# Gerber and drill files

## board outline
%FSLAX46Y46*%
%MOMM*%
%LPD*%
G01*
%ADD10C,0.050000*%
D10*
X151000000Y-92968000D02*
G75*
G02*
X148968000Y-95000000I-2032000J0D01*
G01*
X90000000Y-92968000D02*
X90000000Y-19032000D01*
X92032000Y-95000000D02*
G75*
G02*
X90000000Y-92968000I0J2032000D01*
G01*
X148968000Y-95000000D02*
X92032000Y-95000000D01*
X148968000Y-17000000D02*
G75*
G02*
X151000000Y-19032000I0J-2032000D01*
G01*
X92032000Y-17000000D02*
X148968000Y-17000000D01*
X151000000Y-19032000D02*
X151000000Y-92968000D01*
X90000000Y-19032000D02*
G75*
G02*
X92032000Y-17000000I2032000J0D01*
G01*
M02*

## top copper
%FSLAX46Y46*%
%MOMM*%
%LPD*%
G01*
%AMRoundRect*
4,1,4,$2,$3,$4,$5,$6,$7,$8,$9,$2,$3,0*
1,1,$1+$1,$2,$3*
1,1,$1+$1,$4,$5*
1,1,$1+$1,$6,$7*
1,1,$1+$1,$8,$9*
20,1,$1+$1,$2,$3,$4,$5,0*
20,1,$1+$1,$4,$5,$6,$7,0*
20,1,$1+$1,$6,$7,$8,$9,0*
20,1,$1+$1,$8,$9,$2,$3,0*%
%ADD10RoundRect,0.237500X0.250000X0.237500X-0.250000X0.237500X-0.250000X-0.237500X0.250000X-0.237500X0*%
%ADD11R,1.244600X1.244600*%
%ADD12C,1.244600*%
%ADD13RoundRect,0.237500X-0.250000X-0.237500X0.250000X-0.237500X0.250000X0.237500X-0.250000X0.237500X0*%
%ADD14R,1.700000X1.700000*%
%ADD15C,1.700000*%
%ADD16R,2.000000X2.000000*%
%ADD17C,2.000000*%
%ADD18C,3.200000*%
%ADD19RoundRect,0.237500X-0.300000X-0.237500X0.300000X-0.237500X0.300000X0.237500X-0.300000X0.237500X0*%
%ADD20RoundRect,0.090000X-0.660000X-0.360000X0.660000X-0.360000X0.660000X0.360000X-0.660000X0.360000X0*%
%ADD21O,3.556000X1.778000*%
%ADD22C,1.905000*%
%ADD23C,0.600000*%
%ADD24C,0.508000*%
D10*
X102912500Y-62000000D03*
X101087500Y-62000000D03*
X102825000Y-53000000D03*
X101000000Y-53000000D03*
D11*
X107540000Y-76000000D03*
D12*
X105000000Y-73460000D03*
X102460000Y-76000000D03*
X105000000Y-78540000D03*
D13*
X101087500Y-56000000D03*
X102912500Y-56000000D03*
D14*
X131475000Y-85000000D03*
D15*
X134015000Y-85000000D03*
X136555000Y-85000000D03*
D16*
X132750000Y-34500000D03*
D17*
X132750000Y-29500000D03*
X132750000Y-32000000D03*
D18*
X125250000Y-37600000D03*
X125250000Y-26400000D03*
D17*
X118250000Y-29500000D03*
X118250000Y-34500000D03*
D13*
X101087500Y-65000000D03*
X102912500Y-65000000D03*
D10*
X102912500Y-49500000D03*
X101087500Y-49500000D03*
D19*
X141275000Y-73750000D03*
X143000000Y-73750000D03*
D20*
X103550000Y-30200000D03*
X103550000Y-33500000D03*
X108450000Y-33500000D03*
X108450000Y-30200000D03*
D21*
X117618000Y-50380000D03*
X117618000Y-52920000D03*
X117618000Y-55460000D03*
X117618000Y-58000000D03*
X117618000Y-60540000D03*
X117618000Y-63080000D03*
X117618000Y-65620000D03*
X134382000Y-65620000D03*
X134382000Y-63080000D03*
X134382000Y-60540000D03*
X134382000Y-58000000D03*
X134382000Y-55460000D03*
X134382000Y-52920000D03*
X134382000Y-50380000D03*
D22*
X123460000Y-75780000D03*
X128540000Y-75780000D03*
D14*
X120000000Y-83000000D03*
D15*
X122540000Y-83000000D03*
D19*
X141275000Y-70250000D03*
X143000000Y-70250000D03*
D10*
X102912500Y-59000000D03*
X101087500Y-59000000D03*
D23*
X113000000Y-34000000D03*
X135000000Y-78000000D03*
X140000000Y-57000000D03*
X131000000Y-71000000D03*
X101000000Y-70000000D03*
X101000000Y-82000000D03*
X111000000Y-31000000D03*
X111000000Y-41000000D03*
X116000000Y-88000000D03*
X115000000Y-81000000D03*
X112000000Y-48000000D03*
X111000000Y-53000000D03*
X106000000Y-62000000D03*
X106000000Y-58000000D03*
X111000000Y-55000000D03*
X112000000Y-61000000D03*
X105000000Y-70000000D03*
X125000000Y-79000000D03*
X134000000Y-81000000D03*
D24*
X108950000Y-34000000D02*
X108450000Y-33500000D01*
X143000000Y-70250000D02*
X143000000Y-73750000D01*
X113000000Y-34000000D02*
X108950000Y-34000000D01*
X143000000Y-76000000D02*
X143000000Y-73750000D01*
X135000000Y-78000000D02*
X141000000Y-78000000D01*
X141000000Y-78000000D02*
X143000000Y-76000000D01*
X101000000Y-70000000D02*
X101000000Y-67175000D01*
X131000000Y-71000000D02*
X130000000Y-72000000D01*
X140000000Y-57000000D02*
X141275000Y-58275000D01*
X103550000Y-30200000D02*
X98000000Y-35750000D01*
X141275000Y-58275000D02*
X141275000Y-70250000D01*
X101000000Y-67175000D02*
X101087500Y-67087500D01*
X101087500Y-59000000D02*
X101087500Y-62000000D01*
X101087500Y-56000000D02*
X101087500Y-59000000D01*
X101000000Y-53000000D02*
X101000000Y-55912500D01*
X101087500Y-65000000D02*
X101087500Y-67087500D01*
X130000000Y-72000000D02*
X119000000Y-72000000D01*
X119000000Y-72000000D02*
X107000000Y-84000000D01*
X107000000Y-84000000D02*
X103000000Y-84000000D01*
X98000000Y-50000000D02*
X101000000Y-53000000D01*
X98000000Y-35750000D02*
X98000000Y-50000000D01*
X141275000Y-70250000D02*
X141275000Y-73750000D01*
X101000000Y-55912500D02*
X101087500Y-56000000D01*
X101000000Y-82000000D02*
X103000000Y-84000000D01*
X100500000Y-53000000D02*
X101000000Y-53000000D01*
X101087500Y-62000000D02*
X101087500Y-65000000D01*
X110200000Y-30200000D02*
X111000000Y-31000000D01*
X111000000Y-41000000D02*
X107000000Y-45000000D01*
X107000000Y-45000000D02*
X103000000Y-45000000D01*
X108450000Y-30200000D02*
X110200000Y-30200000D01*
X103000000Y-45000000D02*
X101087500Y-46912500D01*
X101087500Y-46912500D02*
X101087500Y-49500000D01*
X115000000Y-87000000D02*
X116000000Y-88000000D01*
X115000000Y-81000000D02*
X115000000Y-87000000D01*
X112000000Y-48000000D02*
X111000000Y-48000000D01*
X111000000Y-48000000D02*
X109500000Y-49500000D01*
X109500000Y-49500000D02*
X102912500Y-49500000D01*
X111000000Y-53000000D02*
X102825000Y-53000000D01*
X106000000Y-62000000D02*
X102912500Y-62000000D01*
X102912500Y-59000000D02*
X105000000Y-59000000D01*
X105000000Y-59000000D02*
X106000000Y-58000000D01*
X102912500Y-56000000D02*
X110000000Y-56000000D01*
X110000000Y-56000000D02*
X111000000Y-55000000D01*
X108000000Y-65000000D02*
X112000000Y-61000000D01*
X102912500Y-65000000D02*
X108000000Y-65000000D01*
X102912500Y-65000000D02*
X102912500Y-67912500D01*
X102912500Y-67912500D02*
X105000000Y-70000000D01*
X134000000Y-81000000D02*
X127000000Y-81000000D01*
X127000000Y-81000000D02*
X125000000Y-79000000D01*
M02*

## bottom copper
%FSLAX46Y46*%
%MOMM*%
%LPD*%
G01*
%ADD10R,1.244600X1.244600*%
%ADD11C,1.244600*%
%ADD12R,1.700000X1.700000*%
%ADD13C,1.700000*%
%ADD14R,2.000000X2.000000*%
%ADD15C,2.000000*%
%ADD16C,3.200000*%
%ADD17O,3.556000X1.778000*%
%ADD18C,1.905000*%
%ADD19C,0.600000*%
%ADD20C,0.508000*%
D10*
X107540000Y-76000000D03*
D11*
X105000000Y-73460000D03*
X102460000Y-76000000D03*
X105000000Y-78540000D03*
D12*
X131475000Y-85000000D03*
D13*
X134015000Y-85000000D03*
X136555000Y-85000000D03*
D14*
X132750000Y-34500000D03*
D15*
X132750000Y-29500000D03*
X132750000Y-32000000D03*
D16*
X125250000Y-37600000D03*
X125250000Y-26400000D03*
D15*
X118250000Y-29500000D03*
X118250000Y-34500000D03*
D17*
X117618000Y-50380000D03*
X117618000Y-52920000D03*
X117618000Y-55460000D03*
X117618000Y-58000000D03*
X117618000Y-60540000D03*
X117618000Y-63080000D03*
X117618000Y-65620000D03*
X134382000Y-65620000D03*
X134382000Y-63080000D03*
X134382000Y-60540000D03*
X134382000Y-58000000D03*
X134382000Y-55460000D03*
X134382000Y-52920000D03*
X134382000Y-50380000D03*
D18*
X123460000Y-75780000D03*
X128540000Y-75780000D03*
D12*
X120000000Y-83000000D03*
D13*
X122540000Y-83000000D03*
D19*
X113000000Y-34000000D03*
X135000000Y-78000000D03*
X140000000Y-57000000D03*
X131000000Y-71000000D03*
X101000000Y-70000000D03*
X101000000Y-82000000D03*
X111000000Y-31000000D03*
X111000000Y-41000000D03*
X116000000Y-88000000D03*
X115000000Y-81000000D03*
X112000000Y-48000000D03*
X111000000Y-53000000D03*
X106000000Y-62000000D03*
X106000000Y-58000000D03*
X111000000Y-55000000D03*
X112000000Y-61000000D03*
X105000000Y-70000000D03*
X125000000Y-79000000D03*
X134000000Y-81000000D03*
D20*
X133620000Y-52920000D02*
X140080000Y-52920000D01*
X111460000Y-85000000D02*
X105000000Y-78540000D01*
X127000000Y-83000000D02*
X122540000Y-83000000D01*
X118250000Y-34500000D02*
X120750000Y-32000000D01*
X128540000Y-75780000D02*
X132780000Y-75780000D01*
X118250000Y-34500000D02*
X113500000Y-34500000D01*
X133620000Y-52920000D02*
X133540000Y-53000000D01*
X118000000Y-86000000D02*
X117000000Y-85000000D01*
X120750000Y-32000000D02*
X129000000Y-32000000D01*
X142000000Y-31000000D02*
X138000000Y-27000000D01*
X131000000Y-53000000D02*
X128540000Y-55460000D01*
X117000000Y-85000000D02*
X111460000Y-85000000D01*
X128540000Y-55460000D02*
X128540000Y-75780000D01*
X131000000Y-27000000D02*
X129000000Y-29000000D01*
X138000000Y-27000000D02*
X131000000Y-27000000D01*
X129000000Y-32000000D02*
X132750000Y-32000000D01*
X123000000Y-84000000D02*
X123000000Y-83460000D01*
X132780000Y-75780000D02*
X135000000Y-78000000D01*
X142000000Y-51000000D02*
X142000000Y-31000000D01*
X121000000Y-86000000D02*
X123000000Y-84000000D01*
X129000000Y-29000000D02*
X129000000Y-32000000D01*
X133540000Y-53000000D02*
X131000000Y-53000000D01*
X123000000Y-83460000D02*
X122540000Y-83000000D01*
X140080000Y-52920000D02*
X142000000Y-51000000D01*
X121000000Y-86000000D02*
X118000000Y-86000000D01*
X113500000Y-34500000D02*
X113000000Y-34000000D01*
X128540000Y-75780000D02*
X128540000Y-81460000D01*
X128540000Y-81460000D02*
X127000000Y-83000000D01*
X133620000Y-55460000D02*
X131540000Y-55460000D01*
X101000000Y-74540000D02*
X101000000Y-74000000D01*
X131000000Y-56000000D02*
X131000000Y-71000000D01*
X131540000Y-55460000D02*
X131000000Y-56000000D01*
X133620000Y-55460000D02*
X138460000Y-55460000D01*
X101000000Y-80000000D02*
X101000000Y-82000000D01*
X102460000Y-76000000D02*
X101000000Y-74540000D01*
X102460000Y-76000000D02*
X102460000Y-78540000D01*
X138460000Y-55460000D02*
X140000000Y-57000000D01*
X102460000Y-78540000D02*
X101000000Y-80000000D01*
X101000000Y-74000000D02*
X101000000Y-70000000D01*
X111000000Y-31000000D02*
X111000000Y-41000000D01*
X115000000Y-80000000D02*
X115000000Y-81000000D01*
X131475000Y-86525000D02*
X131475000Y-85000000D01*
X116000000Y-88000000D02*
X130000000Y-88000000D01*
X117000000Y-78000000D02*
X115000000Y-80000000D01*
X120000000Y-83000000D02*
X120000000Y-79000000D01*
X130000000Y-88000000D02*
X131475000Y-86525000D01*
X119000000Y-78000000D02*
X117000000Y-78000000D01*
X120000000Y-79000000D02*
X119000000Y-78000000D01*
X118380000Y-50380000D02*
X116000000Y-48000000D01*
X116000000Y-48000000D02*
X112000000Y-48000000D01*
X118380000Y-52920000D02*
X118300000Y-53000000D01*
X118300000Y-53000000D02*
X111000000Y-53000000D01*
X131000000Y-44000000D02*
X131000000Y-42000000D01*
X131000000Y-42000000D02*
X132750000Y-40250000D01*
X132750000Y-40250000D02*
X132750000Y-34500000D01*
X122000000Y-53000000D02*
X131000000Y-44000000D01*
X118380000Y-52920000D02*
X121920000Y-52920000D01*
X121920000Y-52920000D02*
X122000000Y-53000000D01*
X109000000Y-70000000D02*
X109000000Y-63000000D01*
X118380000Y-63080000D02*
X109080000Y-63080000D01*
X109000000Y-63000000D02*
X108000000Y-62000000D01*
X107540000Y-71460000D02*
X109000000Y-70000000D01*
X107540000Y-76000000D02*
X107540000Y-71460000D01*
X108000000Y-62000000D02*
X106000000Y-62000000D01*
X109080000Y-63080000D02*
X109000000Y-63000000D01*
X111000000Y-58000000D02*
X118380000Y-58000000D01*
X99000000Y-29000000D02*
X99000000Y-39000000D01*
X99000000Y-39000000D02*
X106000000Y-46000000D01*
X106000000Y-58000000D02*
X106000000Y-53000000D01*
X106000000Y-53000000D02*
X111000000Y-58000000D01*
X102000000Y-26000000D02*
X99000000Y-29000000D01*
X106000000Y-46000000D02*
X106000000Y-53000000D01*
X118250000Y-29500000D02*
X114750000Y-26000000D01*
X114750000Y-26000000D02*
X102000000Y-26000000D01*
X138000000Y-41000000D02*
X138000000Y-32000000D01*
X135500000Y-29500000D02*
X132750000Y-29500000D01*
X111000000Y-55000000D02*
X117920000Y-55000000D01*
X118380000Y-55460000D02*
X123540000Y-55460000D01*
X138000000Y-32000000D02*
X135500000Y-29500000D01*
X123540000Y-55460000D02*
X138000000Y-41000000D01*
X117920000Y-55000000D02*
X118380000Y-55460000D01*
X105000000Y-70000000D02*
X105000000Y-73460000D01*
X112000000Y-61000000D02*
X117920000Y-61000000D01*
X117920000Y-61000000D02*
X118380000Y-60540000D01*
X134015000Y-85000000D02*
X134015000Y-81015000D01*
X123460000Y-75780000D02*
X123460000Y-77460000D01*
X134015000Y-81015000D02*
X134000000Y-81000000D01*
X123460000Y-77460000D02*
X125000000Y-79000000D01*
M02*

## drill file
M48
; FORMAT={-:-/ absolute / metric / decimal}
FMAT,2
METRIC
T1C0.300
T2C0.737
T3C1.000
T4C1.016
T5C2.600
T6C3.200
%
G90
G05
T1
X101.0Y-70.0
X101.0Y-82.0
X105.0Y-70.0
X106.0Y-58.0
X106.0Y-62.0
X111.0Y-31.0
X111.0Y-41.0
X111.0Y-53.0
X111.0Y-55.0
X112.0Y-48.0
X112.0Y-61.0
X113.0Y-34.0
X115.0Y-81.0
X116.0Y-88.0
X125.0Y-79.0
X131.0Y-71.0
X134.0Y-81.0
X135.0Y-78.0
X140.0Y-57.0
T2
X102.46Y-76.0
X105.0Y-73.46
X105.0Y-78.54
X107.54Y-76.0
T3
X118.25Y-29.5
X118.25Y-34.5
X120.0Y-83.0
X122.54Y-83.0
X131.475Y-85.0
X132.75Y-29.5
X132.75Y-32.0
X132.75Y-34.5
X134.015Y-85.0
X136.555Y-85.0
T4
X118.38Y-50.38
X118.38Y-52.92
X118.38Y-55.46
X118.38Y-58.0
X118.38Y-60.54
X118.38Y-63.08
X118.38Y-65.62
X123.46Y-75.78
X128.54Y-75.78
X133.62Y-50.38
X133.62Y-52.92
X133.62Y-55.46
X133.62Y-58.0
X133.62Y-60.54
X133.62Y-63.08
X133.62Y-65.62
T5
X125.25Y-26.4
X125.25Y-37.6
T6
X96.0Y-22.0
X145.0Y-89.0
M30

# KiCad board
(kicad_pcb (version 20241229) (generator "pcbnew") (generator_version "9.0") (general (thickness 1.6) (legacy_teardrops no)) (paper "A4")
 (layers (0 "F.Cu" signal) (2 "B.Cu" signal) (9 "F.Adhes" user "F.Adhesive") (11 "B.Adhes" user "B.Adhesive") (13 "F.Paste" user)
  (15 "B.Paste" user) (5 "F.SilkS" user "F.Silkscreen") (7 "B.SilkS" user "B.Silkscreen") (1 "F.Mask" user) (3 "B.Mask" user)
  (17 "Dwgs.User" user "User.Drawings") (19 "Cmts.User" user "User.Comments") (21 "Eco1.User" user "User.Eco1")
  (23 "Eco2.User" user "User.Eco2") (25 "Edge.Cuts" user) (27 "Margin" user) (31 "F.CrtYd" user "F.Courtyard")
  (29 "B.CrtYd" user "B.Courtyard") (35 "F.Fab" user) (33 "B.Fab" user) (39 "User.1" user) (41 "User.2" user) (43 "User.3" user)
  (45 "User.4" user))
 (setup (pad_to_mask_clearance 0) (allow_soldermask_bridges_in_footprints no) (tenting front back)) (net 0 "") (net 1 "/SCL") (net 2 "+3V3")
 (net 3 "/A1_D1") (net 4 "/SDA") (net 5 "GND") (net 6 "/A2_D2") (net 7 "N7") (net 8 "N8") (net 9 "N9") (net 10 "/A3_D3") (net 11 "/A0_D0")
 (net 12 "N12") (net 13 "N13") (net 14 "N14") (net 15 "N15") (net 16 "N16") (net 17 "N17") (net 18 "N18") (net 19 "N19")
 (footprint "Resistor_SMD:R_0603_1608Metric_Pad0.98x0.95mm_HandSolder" (layer "F.Cu") (at 102 62 180)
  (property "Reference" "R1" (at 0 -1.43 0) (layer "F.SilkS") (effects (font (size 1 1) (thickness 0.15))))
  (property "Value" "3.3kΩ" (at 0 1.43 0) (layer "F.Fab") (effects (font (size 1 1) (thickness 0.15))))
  (pad "1" smd roundrect (at -0.9125 0 180) (size 0.975 0.95) (layers "F.Cu" "F.Mask" "F.Paste") (roundrect_rratio 0.25) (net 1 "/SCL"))
  (pad "2" smd roundrect (at 0.9125 0 180) (size 0.975 0.95) (layers "F.Cu" "F.Mask" "F.Paste") (roundrect_rratio 0.25) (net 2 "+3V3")))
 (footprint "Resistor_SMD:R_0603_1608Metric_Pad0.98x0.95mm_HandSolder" (layer "F.Cu") (at 101.9125 53 180)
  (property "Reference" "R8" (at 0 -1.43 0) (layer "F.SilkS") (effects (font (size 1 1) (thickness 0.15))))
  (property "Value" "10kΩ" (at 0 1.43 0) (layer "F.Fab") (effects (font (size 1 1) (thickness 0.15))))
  (pad "1" smd roundrect (at -0.9125 0 180) (size 0.975 0.95) (layers "F.Cu" "F.Mask" "F.Paste") (roundrect_rratio 0.25) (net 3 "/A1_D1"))
  (pad "2" smd roundrect (at 0.9125 0 180) (size 0.975 0.95) (layers "F.Cu" "F.Mask" "F.Paste") (roundrect_rratio 0.25) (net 2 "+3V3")))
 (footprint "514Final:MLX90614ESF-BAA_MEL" (layer "F.Cu") (at 107.54 76 90)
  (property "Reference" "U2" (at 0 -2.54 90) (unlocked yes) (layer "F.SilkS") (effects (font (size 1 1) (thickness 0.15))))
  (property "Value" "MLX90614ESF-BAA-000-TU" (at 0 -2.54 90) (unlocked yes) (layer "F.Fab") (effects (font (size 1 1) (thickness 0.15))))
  (pad "1" thru_hole rect (at 0 0 90) (size 1.2446 1.2446) (drill 0.7366) (layers "*.Cu" "*.Mask") (remove_unused_layers no) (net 1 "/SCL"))
  (pad "2" thru_hole circle (at 2.54 -2.54 180) (size 1.2446 1.2446) (drill 0.7366) (layers "*.Cu" "*.Mask") (remove_unused_layers no)
   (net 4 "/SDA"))
  (pad "3" thru_hole circle (at 0 -5.08 90) (size 1.2446 1.2446) (drill 0.7366) (layers "*.Cu" "*.Mask") (remove_unused_layers no)
   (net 2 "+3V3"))
  (pad "4" thru_hole circle (at -2.54 -2.54 180) (size 1.2446 1.2446) (drill 0.7366) (layers "*.Cu" "*.Mask") (remove_unused_layers no)
   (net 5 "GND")))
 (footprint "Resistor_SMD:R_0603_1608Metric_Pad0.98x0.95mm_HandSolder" (layer "F.Cu") (at 102 56)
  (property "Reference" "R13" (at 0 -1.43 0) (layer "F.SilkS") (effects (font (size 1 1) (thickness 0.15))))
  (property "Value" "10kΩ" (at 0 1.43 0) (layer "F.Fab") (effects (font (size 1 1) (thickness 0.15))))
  (pad "1" smd roundrect (at -0.9125 0) (size 0.975 0.95) (layers "F.Cu" "F.Mask" "F.Paste") (roundrect_rratio 0.25) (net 2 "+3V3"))
  (pad "2" smd roundrect (at 0.9125 0) (size 0.975 0.95) (layers "F.Cu" "F.Mask" "F.Paste") (roundrect_rratio 0.25) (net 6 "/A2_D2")))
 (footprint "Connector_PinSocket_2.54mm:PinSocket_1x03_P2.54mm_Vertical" (layer "F.Cu") (at 131.475 85 90)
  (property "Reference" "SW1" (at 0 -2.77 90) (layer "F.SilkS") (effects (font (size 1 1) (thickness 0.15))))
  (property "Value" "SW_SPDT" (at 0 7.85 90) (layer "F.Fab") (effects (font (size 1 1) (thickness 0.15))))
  (pad "1" thru_hole rect (at 0 0 90) (size 1.7 1.7) (drill 1) (layers "*.Cu" "*.Mask") (remove_unused_layers no) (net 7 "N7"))
  (pad "2" thru_hole circle (at 0 2.54 90) (size 1.7 1.7) (drill 1) (layers "*.Cu" "*.Mask") (remove_unused_layers no) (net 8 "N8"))
  (pad "3" thru_hole circle (at 0 5.08 90) (size 1.7 1.7) (drill 1) (layers "*.Cu" "*.Mask") (remove_unused_layers no) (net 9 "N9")))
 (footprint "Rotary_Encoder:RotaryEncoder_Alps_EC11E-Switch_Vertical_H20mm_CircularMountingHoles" (layer "F.Cu") (at 132.75 34.5 180)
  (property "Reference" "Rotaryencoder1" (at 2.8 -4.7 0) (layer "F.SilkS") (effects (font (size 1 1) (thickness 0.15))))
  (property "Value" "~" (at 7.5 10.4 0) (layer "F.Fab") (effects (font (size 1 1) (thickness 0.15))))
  (pad "A" thru_hole rect (at 0 0 180) (size 2 2) (drill 1) (layers "*.Cu" "*.Mask") (remove_unused_layers no) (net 3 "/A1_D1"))
  (pad "B" thru_hole circle (at 0 5 180) (size 2 2) (drill 1) (layers "*.Cu" "*.Mask") (remove_unused_layers no) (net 6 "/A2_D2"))
  (pad "C" thru_hole circle (at 0 2.5 180) (size 2 2) (drill 1) (layers "*.Cu" "*.Mask") (remove_unused_layers no) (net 5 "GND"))
  (pad "MP" thru_hole circle (at 7.5 -3.1 180) (size 3.2 3.2) (drill 2.6) (layers "*.Cu" "*.Mask") (remove_unused_layers no))
  (pad "MP" thru_hole circle (at 7.5 8.1 180) (size 3.2 3.2) (drill 2.6) (layers "*.Cu" "*.Mask") (remove_unused_layers no))
  (pad "S1" thru_hole circle (at 14.5 5 180) (size 2 2) (drill 1) (layers "*.Cu" "*.Mask") (remove_unused_layers no) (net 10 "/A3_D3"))
  (pad "S2" thru_hole circle (at 14.5 0 180) (size 2 2) (drill 1) (layers "*.Cu" "*.Mask") (remove_unused_layers no) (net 5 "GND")))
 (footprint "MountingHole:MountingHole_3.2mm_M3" (layer "F.Cu") (at 145 89)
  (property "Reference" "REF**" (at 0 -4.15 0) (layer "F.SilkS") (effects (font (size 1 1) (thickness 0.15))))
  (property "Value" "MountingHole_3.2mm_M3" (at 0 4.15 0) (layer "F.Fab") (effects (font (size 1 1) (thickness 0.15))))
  (pad "" np_thru_hole circle (at 0 0) (size 3.2 3.2) (drill 3.2) (layers "*.Cu" "*.Mask")))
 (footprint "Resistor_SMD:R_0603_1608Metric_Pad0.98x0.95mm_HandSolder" (layer "F.Cu") (at 102 65)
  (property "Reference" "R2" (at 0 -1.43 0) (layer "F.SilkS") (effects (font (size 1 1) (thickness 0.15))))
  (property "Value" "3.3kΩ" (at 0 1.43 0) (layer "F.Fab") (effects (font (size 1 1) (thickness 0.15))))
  (pad "1" smd roundrect (at -0.9125 0) (size 0.975 0.95) (layers "F.Cu" "F.Mask" "F.Paste") (roundrect_rratio 0.25) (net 2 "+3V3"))
  (pad "2" smd roundrect (at 0.9125 0) (size 0.975 0.95) (layers "F.Cu" "F.Mask" "F.Paste") (roundrect_rratio 0.25) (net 4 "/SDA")))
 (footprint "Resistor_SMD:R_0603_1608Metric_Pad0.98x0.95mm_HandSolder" (layer "F.Cu") (at 102 49.5 180)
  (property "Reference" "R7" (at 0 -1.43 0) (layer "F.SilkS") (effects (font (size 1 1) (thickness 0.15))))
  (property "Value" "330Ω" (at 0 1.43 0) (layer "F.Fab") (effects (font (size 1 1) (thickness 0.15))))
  (pad "1" smd roundrect (at -0.9125 0 180) (size 0.975 0.95) (layers "F.Cu" "F.Mask" "F.Paste") (roundrect_rratio 0.25) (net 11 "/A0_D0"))
  (pad "2" smd roundrect (at 0.9125 0 180) (size 0.975 0.95) (layers "F.Cu" "F.Mask" "F.Paste") (roundrect_rratio 0.25) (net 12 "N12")))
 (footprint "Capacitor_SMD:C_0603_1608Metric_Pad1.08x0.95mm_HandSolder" (layer "F.Cu") (at 142.1375 73.75)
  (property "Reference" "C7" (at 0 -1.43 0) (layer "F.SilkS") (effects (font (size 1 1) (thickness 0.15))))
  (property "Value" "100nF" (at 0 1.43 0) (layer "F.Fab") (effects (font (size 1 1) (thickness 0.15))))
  (pad "1" smd roundrect (at -0.8625 0) (size 1.075 0.95) (layers "F.Cu" "F.Mask" "F.Paste") (roundrect_rratio 0.25) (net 2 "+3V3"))
  (pad "2" smd roundrect (at 0.8625 0) (size 1.075 0.95) (layers "F.Cu" "F.Mask" "F.Paste") (roundrect_rratio 0.25) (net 5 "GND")))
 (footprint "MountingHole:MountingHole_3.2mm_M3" (layer "F.Cu") (at 96 22)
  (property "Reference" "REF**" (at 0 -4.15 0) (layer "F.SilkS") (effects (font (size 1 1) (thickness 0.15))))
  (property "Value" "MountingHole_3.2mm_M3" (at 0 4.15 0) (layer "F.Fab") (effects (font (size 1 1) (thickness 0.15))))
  (pad "" np_thru_hole circle (at 0 0) (size 3.2 3.2) (drill 3.2) (layers "*.Cu" "*.Mask")))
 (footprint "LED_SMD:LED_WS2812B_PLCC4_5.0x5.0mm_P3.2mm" (layer "F.Cu") (at 106 31.85)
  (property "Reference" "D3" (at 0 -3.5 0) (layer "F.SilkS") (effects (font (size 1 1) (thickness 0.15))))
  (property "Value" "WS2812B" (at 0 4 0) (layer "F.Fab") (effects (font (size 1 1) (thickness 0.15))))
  (pad "1" smd roundrect (at -2.45 -1.65) (size 1.5 0.9) (layers "F.Cu" "F.Mask" "F.Paste") (roundrect_rratio 0.1) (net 2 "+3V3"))
  (pad "2" smd roundrect (at -2.45 1.65) (size 1.5 0.9) (layers "F.Cu" "F.Mask" "F.Paste") (roundrect_rratio 0.1) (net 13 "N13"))
  (pad "3" smd roundrect (at 2.45 1.65) (size 1.5 0.9) (layers "F.Cu" "F.Mask" "F.Paste") (roundrect_rratio 0.1) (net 5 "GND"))
  (pad "4" smd roundrect (at 2.45 -1.65) (size 1.5 0.9) (layers "F.Cu" "F.Mask" "F.Paste") (roundrect_rratio 0.1) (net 12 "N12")))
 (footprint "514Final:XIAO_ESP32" (layer "F.Cu") (at 126 58)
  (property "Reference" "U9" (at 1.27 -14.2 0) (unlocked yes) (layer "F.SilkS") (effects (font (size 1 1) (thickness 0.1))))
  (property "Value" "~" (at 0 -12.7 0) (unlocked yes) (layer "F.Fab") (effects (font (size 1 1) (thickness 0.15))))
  (pad "1" thru_hole oval (at -7.62 -7.62) (size 3.556 1.778) (drill 1.016 (offset -0.762 0)) (layers "*.Cu" "*.Mask")
   (remove_unused_layers no) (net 11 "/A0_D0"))
  (pad "2" thru_hole oval (at -7.62 -5.08) (size 3.556 1.778) (drill 1.016 (offset -0.762 0)) (layers "*.Cu" "*.Mask")
   (remove_unused_layers no) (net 3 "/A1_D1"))
  (pad "3" thru_hole oval (at -7.62 -2.54) (size 3.556 1.778) (drill 1.016 (offset -0.762 0)) (layers "*.Cu" "*.Mask")
   (remove_unused_layers no) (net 6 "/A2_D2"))
  (pad "4" thru_hole oval (at -7.62 0) (size 3.556 1.778) (drill 1.016 (offset -0.762 0)) (layers "*.Cu" "*.Mask") (remove_unused_layers no)
   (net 10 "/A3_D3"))
  (pad "5" thru_hole oval (at -7.62 2.54) (size 3.556 1.778) (drill 1.016 (offset -0.762 0)) (layers "*.Cu" "*.Mask")
   (remove_unused_layers no) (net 4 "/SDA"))
  (pad "6" thru_hole oval (at -7.62 5.08) (size 3.556 1.778) (drill 1.016 (offset -0.762 0)) (layers "*.Cu" "*.Mask")
   (remove_unused_layers no) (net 1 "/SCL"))
  (pad "7" thru_hole oval (at -7.62 7.62) (size 3.556 1.778) (drill 1.016 (offset -0.762 0)) (layers "*.Cu" "*.Mask")
   (remove_unused_layers no) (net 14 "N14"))
  (pad "8" thru_hole oval (at 7.62 7.62) (size 3.556 1.778) (drill 1.016 (offset 0.762 0)) (layers "*.Cu" "*.Mask")
   (remove_unused_layers no) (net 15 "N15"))
  (pad "9" thru_hole oval (at 7.62 5.08) (size 3.556 1.778) (drill 1.016 (offset 0.762 0)) (layers "*.Cu" "*.Mask")
   (remove_unused_layers no) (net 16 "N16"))
  (pad "10" thru_hole oval (at 7.62 2.54) (size 3.556 1.778) (drill 1.016 (offset 0.762 0)) (layers "*.Cu" "*.Mask")
   (remove_unused_layers no) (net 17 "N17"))
  (pad "11" thru_hole oval (at 7.62 0) (size 3.556 1.778) (drill 1.016 (offset 0.762 0)) (layers "*.Cu" "*.Mask") (remove_unused_layers no)
   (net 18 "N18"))
  (pad "12" thru_hole oval (at 7.62 -2.54) (size 3.556 1.778) (drill 1.016 (offset 0.762 0)) (layers "*.Cu" "*.Mask")
   (remove_unused_layers no) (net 2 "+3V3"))
  (pad "13" thru_hole oval (at 7.62 -5.08) (size 3.556 1.778) (drill 1.016 (offset 0.762 0)) (layers "*.Cu" "*.Mask")
   (remove_unused_layers no) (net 5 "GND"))
  (pad "14" thru_hole oval (at 7.62 -7.62) (size 3.556 1.778) (drill 1.016 (offset 0.762 0)) (layers "*.Cu" "*.Mask")
   (remove_unused_layers no) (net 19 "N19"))
  (pad "15" thru_hole circle (at -2.54 17.78) (size 1.905 1.905) (drill 1.016) (layers "*.Cu" "*.Mask") (remove_unused_layers no)
   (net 8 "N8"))
  (pad "16" thru_hole circle (at 2.54 17.78) (size 1.905 1.905) (drill 1.016) (layers "*.Cu" "*.Mask") (remove_unused_layers no)
   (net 5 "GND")))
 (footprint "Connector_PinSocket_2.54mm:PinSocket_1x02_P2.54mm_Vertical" (layer "F.Cu") (at 120 83 90)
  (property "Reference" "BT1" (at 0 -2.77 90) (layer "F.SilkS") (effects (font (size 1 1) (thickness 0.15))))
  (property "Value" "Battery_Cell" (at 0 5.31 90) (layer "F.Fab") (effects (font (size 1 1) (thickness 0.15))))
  (pad "1" thru_hole rect (at 0 0 90) (size 1.7 1.7) (drill 1) (layers "*.Cu" "*.Mask") (remove_unused_layers no) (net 7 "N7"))
  (pad "2" thru_hole circle (at 0 2.54 90) (size 1.7 1.7) (drill 1) (layers "*.Cu" "*.Mask") (remove_unused_layers no) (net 5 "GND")))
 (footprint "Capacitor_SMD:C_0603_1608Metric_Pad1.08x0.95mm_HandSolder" (layer "F.Cu") (at 142.1375 70.25)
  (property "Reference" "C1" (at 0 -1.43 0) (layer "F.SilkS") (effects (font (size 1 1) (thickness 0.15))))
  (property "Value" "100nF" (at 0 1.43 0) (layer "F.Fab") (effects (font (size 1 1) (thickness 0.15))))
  (pad "1" smd roundrect (at -0.8625 0) (size 1.075 0.95) (layers "F.Cu" "F.Mask" "F.Paste") (roundrect_rratio 0.25) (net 2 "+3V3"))
  (pad "2" smd roundrect (at 0.8625 0) (size 1.075 0.95) (layers "F.Cu" "F.Mask" "F.Paste") (roundrect_rratio 0.25) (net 5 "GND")))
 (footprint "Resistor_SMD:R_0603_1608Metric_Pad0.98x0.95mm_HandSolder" (layer "F.Cu") (at 102 59 180)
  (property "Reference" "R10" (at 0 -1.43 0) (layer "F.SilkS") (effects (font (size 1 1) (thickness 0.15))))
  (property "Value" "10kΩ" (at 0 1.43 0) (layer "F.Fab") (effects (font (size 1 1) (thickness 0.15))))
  (pad "1" smd roundrect (at -0.9125 0 180) (size 0.975 0.95) (layers "F.Cu" "F.Mask" "F.Paste") (roundrect_rratio 0.25) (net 10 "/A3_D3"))
  (pad "2" smd roundrect (at 0.9125 0 180) (size 0.975 0.95) (layers "F.Cu" "F.Mask" "F.Paste") (roundrect_rratio 0.25) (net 2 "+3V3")))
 (gr_arc (start 151 92.968) (mid 150.404841 94.404841) (end 148.968 95) (stroke (width 0.05) (type default)) (layer "Edge.Cuts"))
 (gr_line (start 90 92.968) (end 90 19.032) (stroke (width 0.05) (type default)) (layer "Edge.Cuts"))
 (gr_arc (start 92.032 95) (mid 90.595159 94.404841) (end 90 92.968) (stroke (width 0.05) (type default)) (layer "Edge.Cuts"))
 (gr_line (start 148.968 95) (end 92.032 95) (stroke (width 0.05) (type default)) (layer "Edge.Cuts"))
 (gr_arc (start 148.968 17) (mid 150.404841 17.595159) (end 151 19.032) (stroke (width 0.05) (type default)) (layer "Edge.Cuts"))
 (gr_line (start 92.032 17) (end 148.968 17) (stroke (width 0.05) (type default)) (layer "Edge.Cuts"))
 (gr_line (start 151 19.032) (end 151 92.968) (stroke (width 0.05) (type default)) (layer "Edge.Cuts"))
 (gr_arc (start 90 19.032) (mid 90.595159 17.595159) (end 92.032 17) (stroke (width 0.05) (type default)) (layer "Edge.Cuts"))
 (segment (start 108.95 34) (end 108.45 33.5) (width 0.508) (layer "F.Cu") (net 5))
 (segment (start 143 70.25) (end 143 73.75) (width 0.508) (layer "F.Cu") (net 5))
 (segment (start 113 34) (end 108.95 34) (width 0.508) (layer "F.Cu") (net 5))
 (segment (start 143 76) (end 143 73.75) (width 0.508) (layer "F.Cu") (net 5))
 (segment (start 135 78) (end 141 78) (width 0.508) (layer "F.Cu") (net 5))
 (segment (start 141 78) (end 143 76) (width 0.508) (layer "F.Cu") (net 5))
 (via (at 113 34) (size 0.6) (drill 0.3) (layers "F.Cu" "B.Cu") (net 5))
 (via (at 135 78) (size 0.6) (drill 0.3) (layers "F.Cu" "B.Cu") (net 5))
 (segment (start 133.62 52.92) (end 140.08 52.92) (width 0.508) (layer "B.Cu") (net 5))
 (segment (start 111.46 85) (end 105 78.54) (width 0.508) (layer "B.Cu") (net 5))
 (segment (start 127 83) (end 122.54 83) (width 0.508) (layer "B.Cu") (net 5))
 (segment (start 118.25 34.5) (end 120.75 32) (width 0.508) (layer "B.Cu") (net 5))
 (segment (start 128.54 75.78) (end 132.78 75.78) (width 0.508) (layer "B.Cu") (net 5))
 (segment (start 118.25 34.5) (end 113.5 34.5) (width 0.508) (layer "B.Cu") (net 5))
 (segment (start 133.62 52.92) (end 133.54 53) (width 0.508) (layer "B.Cu") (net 5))
 (segment (start 118 86) (end 117 85) (width 0.508) (layer "B.Cu") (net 5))
 (segment (start 120.75 32) (end 129 32) (width 0.508) (layer "B.Cu") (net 5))
 (segment (start 142 31) (end 138 27) (width 0.508) (layer "B.Cu") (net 5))
 (segment (start 131 53) (end 128.54 55.46) (width 0.508) (layer "B.Cu") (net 5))
 (segment (start 117 85) (end 111.46 85) (width 0.508) (layer "B.Cu") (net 5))
 (segment (start 128.54 55.46) (end 128.54 75.78) (width 0.508) (layer "B.Cu") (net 5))
 (segment (start 131 27) (end 129 29) (width 0.508) (layer "B.Cu") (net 5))
 (segment (start 138 27) (end 131 27) (width 0.508) (layer "B.Cu") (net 5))
 (segment (start 129 32) (end 132.75 32) (width 0.508) (layer "B.Cu") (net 5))
 (segment (start 123 84) (end 123 83.46) (width 0.508) (layer "B.Cu") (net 5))
 (segment (start 132.78 75.78) (end 135 78) (width 0.508) (layer "B.Cu") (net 5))
 (segment (start 142 51) (end 142 31) (width 0.508) (layer "B.Cu") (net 5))
 (segment (start 121 86) (end 123 84) (width 0.508) (layer "B.Cu") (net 5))
 (segment (start 129 29) (end 129 32) (width 0.508) (layer "B.Cu") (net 5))
 (segment (start 133.54 53) (end 131 53) (width 0.508) (layer "B.Cu") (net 5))
 (segment (start 123 83.46) (end 122.54 83) (width 0.508) (layer "B.Cu") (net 5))
 (segment (start 140.08 52.92) (end 142 51) (width 0.508) (layer "B.Cu") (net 5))
 (segment (start 121 86) (end 118 86) (width 0.508) (layer "B.Cu") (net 5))
 (segment (start 113.5 34.5) (end 113 34) (width 0.508) (layer "B.Cu") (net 5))
 (segment (start 128.54 75.78) (end 128.54 81.46) (width 0.508) (layer "B.Cu") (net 5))
 (segment (start 128.54 81.46) (end 127 83) (width 0.508) (layer "B.Cu") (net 5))
 (segment (start 101 70) (end 101 67.175) (width 0.508) (layer "F.Cu") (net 2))
 (segment (start 131 71) (end 130 72) (width 0.508) (layer "F.Cu") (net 2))
 (segment (start 140 57) (end 141.275 58.275) (width 0.508) (layer "F.Cu") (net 2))
 (segment (start 103.55 30.2) (end 98 35.75) (width 0.508) (layer "F.Cu") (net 2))
 (segment (start 141.275 58.275) (end 141.275 70.25) (width 0.508) (layer "F.Cu") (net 2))
 (segment (start 101 67.175) (end 101.0875 67.0875) (width 0.508) (layer "F.Cu") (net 2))
 (segment (start 101.0875 59) (end 101.0875 62) (width 0.508) (layer "F.Cu") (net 2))
 (segment (start 101.0875 56) (end 101.0875 59) (width 0.508) (layer "F.Cu") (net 2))
 (segment (start 101 53) (end 101 55.9125) (width 0.508) (layer "F.Cu") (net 2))
 (segment (start 101.0875 65) (end 101.0875 67.0875) (width 0.508) (layer "F.Cu") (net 2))
 (segment (start 130 72) (end 119 72) (width 0.508) (layer "F.Cu") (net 2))
 (segment (start 119 72) (end 107 84) (width 0.508) (layer "F.Cu") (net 2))
 (segment (start 107 84) (end 103 84) (width 0.508) (layer "F.Cu") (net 2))
 (segment (start 98 50) (end 101 53) (width 0.508) (layer "F.Cu") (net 2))
 (segment (start 98 35.75) (end 98 50) (width 0.508) (layer "F.Cu") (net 2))
 (segment (start 141.275 70.25) (end 141.275 73.75) (width 0.508) (layer "F.Cu") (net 2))
 (segment (start 101 55.9125) (end 101.0875 56) (width 0.508) (layer "F.Cu") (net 2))
 (segment (start 101 82) (end 103 84) (width 0.508) (layer "F.Cu") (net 2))
 (segment (start 100.5 53) (end 101 53) (width 0.508) (layer "F.Cu") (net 2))
 (segment (start 101.0875 62) (end 101.0875 65) (width 0.508) (layer "F.Cu") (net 2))
 (via (at 140 57) (size 0.6) (drill 0.3) (layers "F.Cu" "B.Cu") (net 2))
 (via (at 131 71) (size 0.6) (drill 0.3) (layers "F.Cu" "B.Cu") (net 2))
 (via (at 101 70) (size 0.6) (drill 0.3) (layers "F.Cu" "B.Cu") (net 2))
 (via (at 101 82) (size 0.6) (drill 0.3) (layers "F.Cu" "B.Cu") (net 2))
 (segment (start 133.62 55.46) (end 131.54 55.46) (width 0.508) (layer "B.Cu") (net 2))
 (segment (start 101 74.54) (end 101 74) (width 0.508) (layer "B.Cu") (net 2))
 (segment (start 131 56) (end 131 71) (width 0.508) (layer "B.Cu") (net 2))
 (segment (start 131.54 55.46) (end 131 56) (width 0.508) (layer "B.Cu") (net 2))
 (segment (start 133.62 55.46) (end 138.46 55.46) (width 0.508) (layer "B.Cu") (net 2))
 (segment (start 101 80) (end 101 82) (width 0.508) (layer "B.Cu") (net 2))
 (segment (start 102.46 76) (end 101 74.54) (width 0.508) (layer "B.Cu") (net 2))
 (segment (start 102.46 76) (end 102.46 78.54) (width 0.508) (layer "B.Cu") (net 2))
 (segment (start 138.46 55.46) (end 140 57) (width 0.508) (layer "B.Cu") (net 2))
 (segment (start 102.46 78.54) (end 101 80) (width 0.508) (layer "B.Cu") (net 2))
 (segment (start 101 74) (end 101 70) (width 0.508) (layer "B.Cu") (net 2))
 (segment (start 110.2 30.2) (end 111 31) (width 0.508) (layer "F.Cu") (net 12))
 (segment (start 111 41) (end 107 45) (width 0.508) (layer "F.Cu") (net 12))
 (segment (start 107 45) (end 103 45) (width 0.508) (layer "F.Cu") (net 12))
 (segment (start 108.45 30.2) (end 110.2 30.2) (width 0.508) (layer "F.Cu") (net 12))
 (segment (start 103 45) (end 101.0875 46.9125) (width 0.508) (layer "F.Cu") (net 12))
 (segment (start 101.0875 46.9125) (end 101.0875 49.5) (width 0.508) (layer "F.Cu") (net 12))
 (via (at 111 31) (size 0.6) (drill 0.3) (layers "F.Cu" "B.Cu") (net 12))
 (via (at 111 41) (size 0.6) (drill 0.3) (layers "F.Cu" "B.Cu") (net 12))
 (segment (start 111 31) (end 111 41) (width 0.508) (layer "B.Cu") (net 12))
 (segment (start 115 87) (end 116 88) (width 0.508) (layer "F.Cu") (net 7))
 (segment (start 115 81) (end 115 87) (width 0.508) (layer "F.Cu") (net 7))
 (via (at 116 88) (size 0.6) (drill 0.3) (layers "F.Cu" "B.Cu") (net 7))
 (via (at 115 81) (size 0.6) (drill 0.3) (layers "F.Cu" "B.Cu") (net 7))
 (segment (start 115 80) (end 115 81) (width 0.508) (layer "B.Cu") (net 7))
 (segment (start 131.475 86.525) (end 131.475 85) (width 0.508) (layer "B.Cu") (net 7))
 (segment (start 116 88) (end 130 88) (width 0.508) (layer "B.Cu") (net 7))
 (segment (start 117 78) (end 115 80) (width 0.508) (layer "B.Cu") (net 7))
 (segment (start 120 83) (end 120 79) (width 0.508) (layer "B.Cu") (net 7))
 (segment (start 130 88) (end 131.475 86.525) (width 0.508) (layer "B.Cu") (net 7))
 (segment (start 119 78) (end 117 78) (width 0.508) (layer "B.Cu") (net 7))
 (segment (start 120 79) (end 119 78) (width 0.508) (layer "B.Cu") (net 7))
 (segment (start 112 48) (end 111 48) (width 0.508) (layer "F.Cu") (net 11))
 (segment (start 111 48) (end 109.5 49.5) (width 0.508) (layer "F.Cu") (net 11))
 (segment (start 109.5 49.5) (end 102.9125 49.5) (width 0.508) (layer "F.Cu") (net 11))
 (via (at 112 48) (size 0.6) (drill 0.3) (layers "F.Cu" "B.Cu") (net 11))
 (segment (start 118.38 50.38) (end 116 48) (width 0.508) (layer "B.Cu") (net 11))
 (segment (start 116 48) (end 112 48) (width 0.508) (layer "B.Cu") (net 11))
 (segment (start 111 53) (end 102.825 53) (width 0.508) (layer "F.Cu") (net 3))
 (via (at 111 53) (size 0.6) (drill 0.3) (layers "F.Cu" "B.Cu") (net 3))
 (segment (start 118.38 52.92) (end 118.3 53) (width 0.508) (layer "B.Cu") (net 3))
 (segment (start 118.3 53) (end 111 53) (width 0.508) (layer "B.Cu") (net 3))
 (segment (start 131 44) (end 131 42) (width 0.508) (layer "B.Cu") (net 3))
 (segment (start 131 42) (end 132.75 40.25) (width 0.508) (layer "B.Cu") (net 3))
 (segment (start 132.75 40.25) (end 132.75 34.5) (width 0.508) (layer "B.Cu") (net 3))
 (segment (start 122 53) (end 131 44) (width 0.508) (layer "B.Cu") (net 3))
 (segment (start 118.38 52.92) (end 121.92 52.92) (width 0.508) (layer "B.Cu") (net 3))
 (segment (start 121.92 52.92) (end 122 53) (width 0.508) (layer "B.Cu") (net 3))
 (segment (start 106 62) (end 102.9125 62) (width 0.508) (layer "F.Cu") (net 1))
 (via (at 106 62) (size 0.6) (drill 0.3) (layers "F.Cu" "B.Cu") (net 1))
 (segment (start 109 70) (end 109 63) (width 0.508) (layer "B.Cu") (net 1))
 (segment (start 118.38 63.08) (end 109.08 63.08) (width 0.508) (layer "B.Cu") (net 1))
 (segment (start 109 63) (end 108 62) (width 0.508) (layer "B.Cu") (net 1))
 (segment (start 107.54 71.46) (end 109 70) (width 0.508) (layer "B.Cu") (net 1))
 (segment (start 107.54 76) (end 107.54 71.46) (width 0.508) (layer "B.Cu") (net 1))
 (segment (start 108 62) (end 106 62) (width 0.508) (layer "B.Cu") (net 1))
 (segment (start 109.08 63.08) (end 109 63) (width 0.508) (layer "B.Cu") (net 1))
 (segment (start 102.9125 59) (end 105 59) (width 0.508) (layer "F.Cu") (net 10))
 (segment (start 105 59) (end 106 58) (width 0.508) (layer "F.Cu") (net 10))
 (via (at 106 58) (size 0.6) (drill 0.3) (layers "F.Cu" "B.Cu") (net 10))
 (segment (start 111 58) (end 118.38 58) (width 0.508) (layer "B.Cu") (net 10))
 (segment (start 99 29) (end 99 39) (width 0.508) (layer "B.Cu") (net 10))
 (segment (start 99 39) (end 106 46) (width 0.508) (layer "B.Cu") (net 10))
 (segment (start 106 58) (end 106 53) (width 0.508) (layer "B.Cu") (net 10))
 (segment (start 106 53) (end 111 58) (width 0.508) (layer "B.Cu") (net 10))
 (segment (start 102 26) (end 99 29) (width 0.508) (layer "B.Cu") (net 10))
 (segment (start 106 46) (end 106 53) (width 0.508) (layer "B.Cu") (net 10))
 (segment (start 118.25 29.5) (end 114.75 26) (width 0.508) (layer "B.Cu") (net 10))
 (segment (start 114.75 26) (end 102 26) (width 0.508) (layer "B.Cu") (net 10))
 (segment (start 102.9125 56) (end 110 56) (width 0.508) (layer "F.Cu") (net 6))
 (segment (start 110 56) (end 111 55) (width 0.508) (layer "F.Cu") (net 6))
 (via (at 111 55) (size 0.6) (drill 0.3) (layers "F.Cu" "B.Cu") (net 6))
 (segment (start 138 41) (end 138 32) (width 0.508) (layer "B.Cu") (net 6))
 (segment (start 135.5 29.5) (end 132.75 29.5) (width 0.508) (layer "B.Cu") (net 6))
 (segment (start 111 55) (end 117.92 55) (width 0.508) (layer "B.Cu") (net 6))
 (segment (start 118.38 55.46) (end 123.54 55.46) (width 0.508) (layer "B.Cu") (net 6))
 (segment (start 138 32) (end 135.5 29.5) (width 0.508) (layer "B.Cu") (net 6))
 (segment (start 123.54 55.46) (end 138 41) (width 0.508) (layer "B.Cu") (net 6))
 (segment (start 117.92 55) (end 118.38 55.46) (width 0.508) (layer "B.Cu") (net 6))
 (segment (start 108 65) (end 112 61) (width 0.508) (layer "F.Cu") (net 4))
 (segment (start 102.9125 65) (end 108 65) (width 0.508) (layer "F.Cu") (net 4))
 (segment (start 102.9125 65) (end 102.9125 67.9125) (width 0.508) (layer "F.Cu") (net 4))
 (segment (start 102.9125 67.9125) (end 105 70) (width 0.508) (layer "F.Cu") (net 4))
 (via (at 112 61) (size 0.6) (drill 0.3) (layers "F.Cu" "B.Cu") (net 4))
 (via (at 105 70) (size 0.6) (drill 0.3) (layers "F.Cu" "B.Cu") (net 4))
 (segment (start 105 70) (end 105 73.46) (width 0.508) (layer "B.Cu") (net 4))
 (segment (start 112 61) (end 117.92 61) (width 0.508) (layer "B.Cu") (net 4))
 (segment (start 117.92 61) (end 118.38 60.54) (width 0.508) (layer "B.Cu") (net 4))
 (segment (start 134 81) (end 127 81) (width 0.508) (layer "F.Cu") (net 8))
 (segment (start 127 81) (end 125 79) (width 0.508) (layer "F.Cu") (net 8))
 (via (at 125 79) (size 0.6) (drill 0.3) (layers "F.Cu" "B.Cu") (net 8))
 (via (at 134 81) (size 0.6) (drill 0.3) (layers "F.Cu" "B.Cu") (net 8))
 (segment (start 134.015 85) (end 134.015 81.015) (width 0.508) (layer "B.Cu") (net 8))
 (segment (start 123.46 75.78) (end 123.46 77.46) (width 0.508) (layer "B.Cu") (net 8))
 (segment (start 134.015 81.015) (end 134 81) (width 0.508) (layer "B.Cu") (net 8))
 (segment (start 123.46 77.46) (end 125 79) (width 0.508) (layer "B.Cu") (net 8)))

